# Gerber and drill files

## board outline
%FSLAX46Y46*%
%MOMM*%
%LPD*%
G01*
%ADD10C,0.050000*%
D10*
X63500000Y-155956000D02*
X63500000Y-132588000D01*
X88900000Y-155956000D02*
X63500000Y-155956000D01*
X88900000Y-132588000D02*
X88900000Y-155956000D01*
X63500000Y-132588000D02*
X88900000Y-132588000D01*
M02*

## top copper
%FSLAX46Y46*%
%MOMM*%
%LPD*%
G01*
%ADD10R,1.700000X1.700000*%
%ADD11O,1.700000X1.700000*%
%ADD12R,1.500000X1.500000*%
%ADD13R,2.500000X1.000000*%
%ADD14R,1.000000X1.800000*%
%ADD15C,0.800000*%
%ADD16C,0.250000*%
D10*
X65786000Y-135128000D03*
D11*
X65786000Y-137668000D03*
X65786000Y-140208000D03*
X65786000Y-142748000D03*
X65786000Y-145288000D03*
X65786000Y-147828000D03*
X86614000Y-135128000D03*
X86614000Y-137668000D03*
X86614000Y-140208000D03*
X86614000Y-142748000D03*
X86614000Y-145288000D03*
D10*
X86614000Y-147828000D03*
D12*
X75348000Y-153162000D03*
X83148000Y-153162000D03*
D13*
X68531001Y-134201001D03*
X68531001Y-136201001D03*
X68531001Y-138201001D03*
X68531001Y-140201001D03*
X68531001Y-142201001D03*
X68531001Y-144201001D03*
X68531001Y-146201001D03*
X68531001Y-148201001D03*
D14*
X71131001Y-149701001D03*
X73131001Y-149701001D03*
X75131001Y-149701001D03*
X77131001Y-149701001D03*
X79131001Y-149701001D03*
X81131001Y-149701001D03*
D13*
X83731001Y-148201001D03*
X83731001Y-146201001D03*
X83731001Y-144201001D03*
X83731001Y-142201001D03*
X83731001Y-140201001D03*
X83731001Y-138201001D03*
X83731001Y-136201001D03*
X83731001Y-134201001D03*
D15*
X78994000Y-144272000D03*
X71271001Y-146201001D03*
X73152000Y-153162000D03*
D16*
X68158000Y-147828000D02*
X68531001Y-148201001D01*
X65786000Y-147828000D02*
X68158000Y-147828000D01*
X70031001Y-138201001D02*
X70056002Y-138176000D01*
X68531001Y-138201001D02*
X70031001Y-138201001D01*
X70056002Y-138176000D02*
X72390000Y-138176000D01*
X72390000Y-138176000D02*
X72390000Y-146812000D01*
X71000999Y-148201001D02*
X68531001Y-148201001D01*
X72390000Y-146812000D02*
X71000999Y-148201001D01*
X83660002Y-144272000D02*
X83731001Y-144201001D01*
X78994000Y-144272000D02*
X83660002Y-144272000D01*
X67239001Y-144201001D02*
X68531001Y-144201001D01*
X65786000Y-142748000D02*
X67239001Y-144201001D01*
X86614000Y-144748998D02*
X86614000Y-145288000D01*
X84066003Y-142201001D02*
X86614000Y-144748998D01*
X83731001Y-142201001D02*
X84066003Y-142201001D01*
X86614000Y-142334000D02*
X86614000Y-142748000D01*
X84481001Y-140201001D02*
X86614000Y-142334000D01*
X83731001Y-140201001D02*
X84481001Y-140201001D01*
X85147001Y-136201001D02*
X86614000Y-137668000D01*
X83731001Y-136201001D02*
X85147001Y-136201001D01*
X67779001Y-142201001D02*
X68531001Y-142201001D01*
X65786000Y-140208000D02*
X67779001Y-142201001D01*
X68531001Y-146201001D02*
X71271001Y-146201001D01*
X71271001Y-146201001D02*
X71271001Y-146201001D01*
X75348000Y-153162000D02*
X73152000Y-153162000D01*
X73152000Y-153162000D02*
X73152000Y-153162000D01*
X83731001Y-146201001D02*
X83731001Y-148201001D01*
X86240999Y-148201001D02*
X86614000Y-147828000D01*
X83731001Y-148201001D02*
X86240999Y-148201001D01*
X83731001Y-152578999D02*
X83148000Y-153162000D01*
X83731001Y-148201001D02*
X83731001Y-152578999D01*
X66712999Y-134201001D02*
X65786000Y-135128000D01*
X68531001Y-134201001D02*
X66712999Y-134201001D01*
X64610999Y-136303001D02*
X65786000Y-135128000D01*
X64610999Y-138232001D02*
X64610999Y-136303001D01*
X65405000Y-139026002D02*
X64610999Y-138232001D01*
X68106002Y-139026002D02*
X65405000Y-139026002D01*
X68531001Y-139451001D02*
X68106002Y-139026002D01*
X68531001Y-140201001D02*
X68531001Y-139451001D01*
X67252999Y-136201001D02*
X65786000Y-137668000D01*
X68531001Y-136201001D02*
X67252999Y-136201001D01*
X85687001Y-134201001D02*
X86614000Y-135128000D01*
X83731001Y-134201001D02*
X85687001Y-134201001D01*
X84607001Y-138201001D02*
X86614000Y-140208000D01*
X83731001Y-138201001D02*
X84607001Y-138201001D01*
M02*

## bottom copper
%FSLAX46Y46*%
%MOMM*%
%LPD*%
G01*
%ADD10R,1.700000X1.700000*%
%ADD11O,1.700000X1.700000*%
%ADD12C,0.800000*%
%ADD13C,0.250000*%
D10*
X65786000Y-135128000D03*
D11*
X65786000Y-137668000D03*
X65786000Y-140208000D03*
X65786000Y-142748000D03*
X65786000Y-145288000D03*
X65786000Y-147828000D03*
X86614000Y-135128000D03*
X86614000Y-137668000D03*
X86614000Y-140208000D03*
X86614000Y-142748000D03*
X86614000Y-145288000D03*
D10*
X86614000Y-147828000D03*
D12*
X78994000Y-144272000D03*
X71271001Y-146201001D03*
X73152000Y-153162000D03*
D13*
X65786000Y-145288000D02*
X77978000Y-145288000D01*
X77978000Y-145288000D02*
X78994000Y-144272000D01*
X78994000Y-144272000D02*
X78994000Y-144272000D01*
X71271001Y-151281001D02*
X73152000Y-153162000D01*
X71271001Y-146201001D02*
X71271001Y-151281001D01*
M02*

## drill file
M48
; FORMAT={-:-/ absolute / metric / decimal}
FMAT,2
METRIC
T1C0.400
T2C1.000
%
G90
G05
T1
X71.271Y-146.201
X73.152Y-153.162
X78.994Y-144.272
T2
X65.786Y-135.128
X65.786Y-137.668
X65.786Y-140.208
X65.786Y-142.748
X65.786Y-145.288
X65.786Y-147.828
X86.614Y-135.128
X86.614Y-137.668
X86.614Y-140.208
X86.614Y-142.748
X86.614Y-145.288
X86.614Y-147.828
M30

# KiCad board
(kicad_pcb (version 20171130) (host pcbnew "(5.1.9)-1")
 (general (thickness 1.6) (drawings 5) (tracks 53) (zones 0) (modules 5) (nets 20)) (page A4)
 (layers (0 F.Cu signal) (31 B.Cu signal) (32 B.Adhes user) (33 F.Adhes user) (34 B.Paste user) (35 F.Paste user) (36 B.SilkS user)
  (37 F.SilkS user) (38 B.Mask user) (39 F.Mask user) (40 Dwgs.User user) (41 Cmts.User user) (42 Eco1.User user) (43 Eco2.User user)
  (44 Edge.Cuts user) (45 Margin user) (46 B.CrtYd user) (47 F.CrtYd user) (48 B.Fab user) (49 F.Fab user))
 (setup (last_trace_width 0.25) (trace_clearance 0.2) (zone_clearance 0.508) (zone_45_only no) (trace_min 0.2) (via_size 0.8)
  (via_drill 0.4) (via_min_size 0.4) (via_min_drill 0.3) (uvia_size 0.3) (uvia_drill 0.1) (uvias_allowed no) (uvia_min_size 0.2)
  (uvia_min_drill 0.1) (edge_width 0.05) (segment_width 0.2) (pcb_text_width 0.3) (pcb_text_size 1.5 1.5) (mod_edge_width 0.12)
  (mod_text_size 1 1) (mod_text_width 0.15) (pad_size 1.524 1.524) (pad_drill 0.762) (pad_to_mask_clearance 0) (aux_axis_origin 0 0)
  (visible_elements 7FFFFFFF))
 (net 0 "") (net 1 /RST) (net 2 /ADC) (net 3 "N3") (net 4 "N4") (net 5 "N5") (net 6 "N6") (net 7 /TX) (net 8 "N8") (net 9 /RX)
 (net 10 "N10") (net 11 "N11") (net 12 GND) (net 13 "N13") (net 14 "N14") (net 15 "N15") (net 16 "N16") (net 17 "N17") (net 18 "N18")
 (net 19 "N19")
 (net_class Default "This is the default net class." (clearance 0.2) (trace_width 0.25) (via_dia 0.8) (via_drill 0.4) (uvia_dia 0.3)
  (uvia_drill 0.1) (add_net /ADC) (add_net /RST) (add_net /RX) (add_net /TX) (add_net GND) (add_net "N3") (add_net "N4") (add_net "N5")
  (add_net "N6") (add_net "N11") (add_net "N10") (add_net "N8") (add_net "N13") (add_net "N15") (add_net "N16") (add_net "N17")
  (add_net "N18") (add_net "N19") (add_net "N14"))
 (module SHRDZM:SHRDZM (layer F.Cu) (at 68.072 153.416)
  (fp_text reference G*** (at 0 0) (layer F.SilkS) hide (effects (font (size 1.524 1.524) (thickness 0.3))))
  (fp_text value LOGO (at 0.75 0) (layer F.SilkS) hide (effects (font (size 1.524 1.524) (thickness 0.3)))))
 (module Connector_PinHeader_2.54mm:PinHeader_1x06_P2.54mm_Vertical (layer B.Cu) (at 65.786 135.128 180)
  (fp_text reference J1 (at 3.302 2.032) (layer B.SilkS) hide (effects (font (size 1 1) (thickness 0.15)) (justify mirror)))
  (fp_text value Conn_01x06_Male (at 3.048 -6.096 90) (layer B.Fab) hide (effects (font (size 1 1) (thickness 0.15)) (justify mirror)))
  (pad 1 thru_hole rect (at 0 0 180) (size 1.7 1.7) (drill 1) (layers *.Cu *.Mask) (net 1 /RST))
  (pad 2 thru_hole oval (at 0 -2.54 180) (size 1.7 1.7) (drill 1) (layers *.Cu *.Mask) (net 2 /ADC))
  (pad 3 thru_hole oval (at 0 -5.08 180) (size 1.7 1.7) (drill 1) (layers *.Cu *.Mask) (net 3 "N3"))
  (pad 4 thru_hole oval (at 0 -7.62 180) (size 1.7 1.7) (drill 1) (layers *.Cu *.Mask) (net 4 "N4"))
  (pad 5 thru_hole oval (at 0 -10.16 180) (size 1.7 1.7) (drill 1) (layers *.Cu *.Mask) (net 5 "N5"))
  (pad 6 thru_hole oval (at 0 -12.7 180) (size 1.7 1.7) (drill 1) (layers *.Cu *.Mask) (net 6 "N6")))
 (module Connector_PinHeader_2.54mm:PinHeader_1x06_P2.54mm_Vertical (layer B.Cu) (at 86.614 147.828)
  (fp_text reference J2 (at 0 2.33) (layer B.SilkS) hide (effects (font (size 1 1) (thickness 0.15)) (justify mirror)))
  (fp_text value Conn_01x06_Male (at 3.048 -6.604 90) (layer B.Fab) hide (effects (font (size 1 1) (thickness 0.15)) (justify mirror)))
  (pad 6 thru_hole oval (at 0 -12.7) (size 1.7 1.7) (drill 1) (layers *.Cu *.Mask) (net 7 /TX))
  (pad 5 thru_hole oval (at 0 -10.16) (size 1.7 1.7) (drill 1) (layers *.Cu *.Mask) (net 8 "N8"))
  (pad 4 thru_hole oval (at 0 -7.62) (size 1.7 1.7) (drill 1) (layers *.Cu *.Mask) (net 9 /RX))
  (pad 3 thru_hole oval (at 0 -5.08) (size 1.7 1.7) (drill 1) (layers *.Cu *.Mask) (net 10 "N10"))
  (pad 2 thru_hole oval (at 0 -2.54) (size 1.7 1.7) (drill 1) (layers *.Cu *.Mask) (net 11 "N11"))
  (pad 1 thru_hole rect (at 0 0) (size 1.7 1.7) (drill 1) (layers *.Cu *.Mask) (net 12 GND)))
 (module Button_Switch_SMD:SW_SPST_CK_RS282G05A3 (layer F.Cu) (at 79.248 153.162)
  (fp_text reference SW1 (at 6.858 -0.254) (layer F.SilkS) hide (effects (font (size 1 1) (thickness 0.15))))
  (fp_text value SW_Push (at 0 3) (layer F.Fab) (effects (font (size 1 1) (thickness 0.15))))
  (pad 1 smd rect (at -3.9 0) (size 1.5 1.5) (layers F.Cu F.Paste F.Mask) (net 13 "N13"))
  (pad 2 smd rect (at 3.9 0) (size 1.5 1.5) (layers F.Cu F.Paste F.Mask) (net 12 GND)))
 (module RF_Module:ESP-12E (layer F.Cu) (at 76.131001 137.701001)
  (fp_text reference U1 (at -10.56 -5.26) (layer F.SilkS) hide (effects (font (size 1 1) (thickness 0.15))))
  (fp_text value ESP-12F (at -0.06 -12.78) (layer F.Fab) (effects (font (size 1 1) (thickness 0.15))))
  (pad 1 smd rect (at -7.6 -3.5) (size 2.5 1) (layers F.Cu F.Paste F.Mask) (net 1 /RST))
  (pad 2 smd rect (at -7.6 -1.5) (size 2.5 1) (layers F.Cu F.Paste F.Mask) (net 2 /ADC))
  (pad 3 smd rect (at -7.6 0.5) (size 2.5 1) (layers F.Cu F.Paste F.Mask) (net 6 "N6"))
  (pad 4 smd rect (at -7.6 2.5) (size 2.5 1) (layers F.Cu F.Paste F.Mask) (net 1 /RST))
  (pad 5 smd rect (at -7.6 4.5) (size 2.5 1) (layers F.Cu F.Paste F.Mask) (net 3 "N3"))
  (pad 6 smd rect (at -7.6 6.5) (size 2.5 1) (layers F.Cu F.Paste F.Mask) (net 4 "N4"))
  (pad 7 smd rect (at -7.6 8.5) (size 2.5 1) (layers F.Cu F.Paste F.Mask) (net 13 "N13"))
  (pad 8 smd rect (at -7.6 10.5) (size 2.5 1) (layers F.Cu F.Paste F.Mask) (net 6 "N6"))
  (pad 9 smd rect (at -5 12) (size 1 1.8) (layers F.Cu F.Paste F.Mask) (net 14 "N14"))
  (pad 10 smd rect (at -3 12) (size 1 1.8) (layers F.Cu F.Paste F.Mask) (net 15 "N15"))
  (pad 11 smd rect (at -1 12) (size 1 1.8) (layers F.Cu F.Paste F.Mask) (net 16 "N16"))
  (pad 12 smd rect (at 1 12) (size 1 1.8) (layers F.Cu F.Paste F.Mask) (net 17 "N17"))
  (pad 13 smd rect (at 3 12) (size 1 1.8) (layers F.Cu F.Paste F.Mask) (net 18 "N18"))
  (pad 14 smd rect (at 5 12) (size 1 1.8) (layers F.Cu F.Paste F.Mask) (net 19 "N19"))
  (pad 15 smd rect (at 7.6 10.5) (size 2.5 1) (layers F.Cu F.Paste F.Mask) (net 12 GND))
  (pad 16 smd rect (at 7.6 8.5) (size 2.5 1) (layers F.Cu F.Paste F.Mask) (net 12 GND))
  (pad 17 smd rect (at 7.6 6.5) (size 2.5 1) (layers F.Cu F.Paste F.Mask) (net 5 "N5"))
  (pad 18 smd rect (at 7.6 4.5) (size 2.5 1) (layers F.Cu F.Paste F.Mask) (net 11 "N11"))
  (pad 19 smd rect (at 7.6 2.5) (size 2.5 1) (layers F.Cu F.Paste F.Mask) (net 10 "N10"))
  (pad 20 smd rect (at 7.6 0.5) (size 2.5 1) (layers F.Cu F.Paste F.Mask) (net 9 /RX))
  (pad 21 smd rect (at 7.6 -1.5) (size 2.5 1) (layers F.Cu F.Paste F.Mask) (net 8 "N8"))
  (pad 22 smd rect (at 7.6 -3.5) (size 2.5 1) (layers F.Cu F.Paste F.Mask) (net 7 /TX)))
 (gr_line (start 63.5 155.956) (end 63.5 132.588) (layer Edge.Cuts) (width 0.05))
 (gr_line (start 88.9 155.956) (end 63.5 155.956) (layer Edge.Cuts) (width 0.05))
 (gr_line (start 88.9 132.588) (end 88.9 155.956) (layer Edge.Cuts) (width 0.05))
 (gr_line (start 63.5 132.588) (end 88.9 132.588) (layer Edge.Cuts) (width 0.05))
 (segment (start 68.158 147.828) (end 68.531001 148.201001) (width 0.25) (layer F.Cu) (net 6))
 (segment (start 65.786 147.828) (end 68.158 147.828) (width 0.25) (layer F.Cu) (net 6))
 (segment (start 70.031001 138.201001) (end 70.056002 138.176) (width 0.25) (layer F.Cu) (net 6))
 (segment (start 68.531001 138.201001) (end 70.031001 138.201001) (width 0.25) (layer F.Cu) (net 6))
 (segment (start 70.056002 138.176) (end 72.39 138.176) (width 0.25) (layer F.Cu) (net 6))
 (segment (start 72.39 138.176) (end 72.39 146.812) (width 0.25) (layer F.Cu) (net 6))
 (segment (start 71.000999 148.201001) (end 68.531001 148.201001) (width 0.25) (layer F.Cu) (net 6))
 (segment (start 72.39 146.812) (end 71.000999 148.201001) (width 0.25) (layer F.Cu) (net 6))
 (segment (start 65.786 145.288) (end 77.978 145.288) (width 0.25) (layer B.Cu) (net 5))
 (segment (start 77.978 145.288) (end 78.994 144.272) (width 0.25) (layer B.Cu) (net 5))
 (segment (start 78.994 144.272) (end 78.994 144.272) (width 0.25) (layer B.Cu) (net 5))
 (via (at 78.994 144.272) (size 0.8) (drill 0.4) (layers F.Cu B.Cu) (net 5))
 (segment (start 83.660002 144.272) (end 83.731001 144.201001) (width 0.25) (layer F.Cu) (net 5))
 (segment (start 78.994 144.272) (end 83.660002 144.272) (width 0.25) (layer F.Cu) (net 5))
 (segment (start 67.239001 144.201001) (end 68.531001 144.201001) (width 0.25) (layer F.Cu) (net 4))
 (segment (start 65.786 142.748) (end 67.239001 144.201001) (width 0.25) (layer F.Cu) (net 4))
 (segment (start 86.614 144.748998) (end 86.614 145.288) (width 0.25) (layer F.Cu) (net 11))
 (segment (start 84.066003 142.201001) (end 86.614 144.748998) (width 0.25) (layer F.Cu) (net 11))
 (segment (start 83.731001 142.201001) (end 84.066003 142.201001) (width 0.25) (layer F.Cu) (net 11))
 (segment (start 86.614 142.334) (end 86.614 142.748) (width 0.25) (layer F.Cu) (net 10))
 (segment (start 84.481001 140.201001) (end 86.614 142.334) (width 0.25) (layer F.Cu) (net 10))
 (segment (start 83.731001 140.201001) (end 84.481001 140.201001) (width 0.25) (layer F.Cu) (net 10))
 (segment (start 85.147001 136.201001) (end 86.614 137.668) (width 0.25) (layer F.Cu) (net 8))
 (segment (start 83.731001 136.201001) (end 85.147001 136.201001) (width 0.25) (layer F.Cu) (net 8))
 (segment (start 67.779001 142.201001) (end 68.531001 142.201001) (width 0.25) (layer F.Cu) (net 3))
 (segment (start 65.786 140.208) (end 67.779001 142.201001) (width 0.25) (layer F.Cu) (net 3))
 (segment (start 68.531001 146.201001) (end 71.271001 146.201001) (width 0.25) (layer F.Cu) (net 13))
 (segment (start 71.271001 146.201001) (end 71.271001 146.201001) (width 0.25) (layer F.Cu) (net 13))
 (via (at 71.271001 146.201001) (size 0.8) (drill 0.4) (layers F.Cu B.Cu) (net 13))
 (segment (start 75.348 153.162) (end 73.152 153.162) (width 0.25) (layer F.Cu) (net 13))
 (segment (start 73.152 153.162) (end 73.152 153.162) (width 0.25) (layer F.Cu) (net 13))
 (via (at 73.152 153.162) (size 0.8) (drill 0.4) (layers F.Cu B.Cu) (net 13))
 (segment (start 71.271001 151.281001) (end 73.152 153.162) (width 0.25) (layer B.Cu) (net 13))
 (segment (start 71.271001 146.201001) (end 71.271001 151.281001) (width 0.25) (layer B.Cu) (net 13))
 (segment (start 83.731001 146.201001) (end 83.731001 148.201001) (width 0.25) (layer F.Cu) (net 12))
 (segment (start 86.240999 148.201001) (end 86.614 147.828) (width 0.25) (layer F.Cu) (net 12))
 (segment (start 83.731001 148.201001) (end 86.240999 148.201001) (width 0.25) (layer F.Cu) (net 12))
 (segment (start 83.731001 152.578999) (end 83.148 153.162) (width 0.25) (layer F.Cu) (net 12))
 (segment (start 83.731001 148.201001) (end 83.731001 152.578999) (width 0.25) (layer F.Cu) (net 12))
 (segment (start 66.712999 134.201001) (end 65.786 135.128) (width 0.25) (layer F.Cu) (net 1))
 (segment (start 68.531001 134.201001) (end 66.712999 134.201001) (width 0.25) (layer F.Cu) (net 1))
 (segment (start 64.610999 136.303001) (end 65.786 135.128) (width 0.25) (layer F.Cu) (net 1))
 (segment (start 64.610999 138.232001) (end 64.610999 136.303001) (width 0.25) (layer F.Cu) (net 1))
 (segment (start 65.405 139.026002) (end 64.610999 138.232001) (width 0.25) (layer F.Cu) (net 1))
 (segment (start 68.106002 139.026002) (end 65.405 139.026002) (width 0.25) (layer F.Cu) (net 1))
 (segment (start 68.531001 139.451001) (end 68.106002 139.026002) (width 0.25) (layer F.Cu) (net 1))
 (segment (start 68.531001 140.201001) (end 68.531001 139.451001) (width 0.25) (layer F.Cu) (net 1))
 (segment (start 67.252999 136.201001) (end 65.786 137.668) (width 0.25) (layer F.Cu) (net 2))
 (segment (start 68.531001 136.201001) (end 67.252999 136.201001) (width 0.25) (layer F.Cu) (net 2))
 (segment (start 85.687001 134.201001) (end 86.614 135.128) (width 0.25) (layer F.Cu) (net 7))
 (segment (start 83.731001 134.201001) (end 85.687001 134.201001) (width 0.25) (layer F.Cu) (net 7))
 (segment (start 84.607001 138.201001) (end 86.614 140.208) (width 0.25) (layer F.Cu) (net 9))
 (segment (start 83.731001 138.201001) (end 84.607001 138.201001) (width 0.25) (layer F.Cu) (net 9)))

